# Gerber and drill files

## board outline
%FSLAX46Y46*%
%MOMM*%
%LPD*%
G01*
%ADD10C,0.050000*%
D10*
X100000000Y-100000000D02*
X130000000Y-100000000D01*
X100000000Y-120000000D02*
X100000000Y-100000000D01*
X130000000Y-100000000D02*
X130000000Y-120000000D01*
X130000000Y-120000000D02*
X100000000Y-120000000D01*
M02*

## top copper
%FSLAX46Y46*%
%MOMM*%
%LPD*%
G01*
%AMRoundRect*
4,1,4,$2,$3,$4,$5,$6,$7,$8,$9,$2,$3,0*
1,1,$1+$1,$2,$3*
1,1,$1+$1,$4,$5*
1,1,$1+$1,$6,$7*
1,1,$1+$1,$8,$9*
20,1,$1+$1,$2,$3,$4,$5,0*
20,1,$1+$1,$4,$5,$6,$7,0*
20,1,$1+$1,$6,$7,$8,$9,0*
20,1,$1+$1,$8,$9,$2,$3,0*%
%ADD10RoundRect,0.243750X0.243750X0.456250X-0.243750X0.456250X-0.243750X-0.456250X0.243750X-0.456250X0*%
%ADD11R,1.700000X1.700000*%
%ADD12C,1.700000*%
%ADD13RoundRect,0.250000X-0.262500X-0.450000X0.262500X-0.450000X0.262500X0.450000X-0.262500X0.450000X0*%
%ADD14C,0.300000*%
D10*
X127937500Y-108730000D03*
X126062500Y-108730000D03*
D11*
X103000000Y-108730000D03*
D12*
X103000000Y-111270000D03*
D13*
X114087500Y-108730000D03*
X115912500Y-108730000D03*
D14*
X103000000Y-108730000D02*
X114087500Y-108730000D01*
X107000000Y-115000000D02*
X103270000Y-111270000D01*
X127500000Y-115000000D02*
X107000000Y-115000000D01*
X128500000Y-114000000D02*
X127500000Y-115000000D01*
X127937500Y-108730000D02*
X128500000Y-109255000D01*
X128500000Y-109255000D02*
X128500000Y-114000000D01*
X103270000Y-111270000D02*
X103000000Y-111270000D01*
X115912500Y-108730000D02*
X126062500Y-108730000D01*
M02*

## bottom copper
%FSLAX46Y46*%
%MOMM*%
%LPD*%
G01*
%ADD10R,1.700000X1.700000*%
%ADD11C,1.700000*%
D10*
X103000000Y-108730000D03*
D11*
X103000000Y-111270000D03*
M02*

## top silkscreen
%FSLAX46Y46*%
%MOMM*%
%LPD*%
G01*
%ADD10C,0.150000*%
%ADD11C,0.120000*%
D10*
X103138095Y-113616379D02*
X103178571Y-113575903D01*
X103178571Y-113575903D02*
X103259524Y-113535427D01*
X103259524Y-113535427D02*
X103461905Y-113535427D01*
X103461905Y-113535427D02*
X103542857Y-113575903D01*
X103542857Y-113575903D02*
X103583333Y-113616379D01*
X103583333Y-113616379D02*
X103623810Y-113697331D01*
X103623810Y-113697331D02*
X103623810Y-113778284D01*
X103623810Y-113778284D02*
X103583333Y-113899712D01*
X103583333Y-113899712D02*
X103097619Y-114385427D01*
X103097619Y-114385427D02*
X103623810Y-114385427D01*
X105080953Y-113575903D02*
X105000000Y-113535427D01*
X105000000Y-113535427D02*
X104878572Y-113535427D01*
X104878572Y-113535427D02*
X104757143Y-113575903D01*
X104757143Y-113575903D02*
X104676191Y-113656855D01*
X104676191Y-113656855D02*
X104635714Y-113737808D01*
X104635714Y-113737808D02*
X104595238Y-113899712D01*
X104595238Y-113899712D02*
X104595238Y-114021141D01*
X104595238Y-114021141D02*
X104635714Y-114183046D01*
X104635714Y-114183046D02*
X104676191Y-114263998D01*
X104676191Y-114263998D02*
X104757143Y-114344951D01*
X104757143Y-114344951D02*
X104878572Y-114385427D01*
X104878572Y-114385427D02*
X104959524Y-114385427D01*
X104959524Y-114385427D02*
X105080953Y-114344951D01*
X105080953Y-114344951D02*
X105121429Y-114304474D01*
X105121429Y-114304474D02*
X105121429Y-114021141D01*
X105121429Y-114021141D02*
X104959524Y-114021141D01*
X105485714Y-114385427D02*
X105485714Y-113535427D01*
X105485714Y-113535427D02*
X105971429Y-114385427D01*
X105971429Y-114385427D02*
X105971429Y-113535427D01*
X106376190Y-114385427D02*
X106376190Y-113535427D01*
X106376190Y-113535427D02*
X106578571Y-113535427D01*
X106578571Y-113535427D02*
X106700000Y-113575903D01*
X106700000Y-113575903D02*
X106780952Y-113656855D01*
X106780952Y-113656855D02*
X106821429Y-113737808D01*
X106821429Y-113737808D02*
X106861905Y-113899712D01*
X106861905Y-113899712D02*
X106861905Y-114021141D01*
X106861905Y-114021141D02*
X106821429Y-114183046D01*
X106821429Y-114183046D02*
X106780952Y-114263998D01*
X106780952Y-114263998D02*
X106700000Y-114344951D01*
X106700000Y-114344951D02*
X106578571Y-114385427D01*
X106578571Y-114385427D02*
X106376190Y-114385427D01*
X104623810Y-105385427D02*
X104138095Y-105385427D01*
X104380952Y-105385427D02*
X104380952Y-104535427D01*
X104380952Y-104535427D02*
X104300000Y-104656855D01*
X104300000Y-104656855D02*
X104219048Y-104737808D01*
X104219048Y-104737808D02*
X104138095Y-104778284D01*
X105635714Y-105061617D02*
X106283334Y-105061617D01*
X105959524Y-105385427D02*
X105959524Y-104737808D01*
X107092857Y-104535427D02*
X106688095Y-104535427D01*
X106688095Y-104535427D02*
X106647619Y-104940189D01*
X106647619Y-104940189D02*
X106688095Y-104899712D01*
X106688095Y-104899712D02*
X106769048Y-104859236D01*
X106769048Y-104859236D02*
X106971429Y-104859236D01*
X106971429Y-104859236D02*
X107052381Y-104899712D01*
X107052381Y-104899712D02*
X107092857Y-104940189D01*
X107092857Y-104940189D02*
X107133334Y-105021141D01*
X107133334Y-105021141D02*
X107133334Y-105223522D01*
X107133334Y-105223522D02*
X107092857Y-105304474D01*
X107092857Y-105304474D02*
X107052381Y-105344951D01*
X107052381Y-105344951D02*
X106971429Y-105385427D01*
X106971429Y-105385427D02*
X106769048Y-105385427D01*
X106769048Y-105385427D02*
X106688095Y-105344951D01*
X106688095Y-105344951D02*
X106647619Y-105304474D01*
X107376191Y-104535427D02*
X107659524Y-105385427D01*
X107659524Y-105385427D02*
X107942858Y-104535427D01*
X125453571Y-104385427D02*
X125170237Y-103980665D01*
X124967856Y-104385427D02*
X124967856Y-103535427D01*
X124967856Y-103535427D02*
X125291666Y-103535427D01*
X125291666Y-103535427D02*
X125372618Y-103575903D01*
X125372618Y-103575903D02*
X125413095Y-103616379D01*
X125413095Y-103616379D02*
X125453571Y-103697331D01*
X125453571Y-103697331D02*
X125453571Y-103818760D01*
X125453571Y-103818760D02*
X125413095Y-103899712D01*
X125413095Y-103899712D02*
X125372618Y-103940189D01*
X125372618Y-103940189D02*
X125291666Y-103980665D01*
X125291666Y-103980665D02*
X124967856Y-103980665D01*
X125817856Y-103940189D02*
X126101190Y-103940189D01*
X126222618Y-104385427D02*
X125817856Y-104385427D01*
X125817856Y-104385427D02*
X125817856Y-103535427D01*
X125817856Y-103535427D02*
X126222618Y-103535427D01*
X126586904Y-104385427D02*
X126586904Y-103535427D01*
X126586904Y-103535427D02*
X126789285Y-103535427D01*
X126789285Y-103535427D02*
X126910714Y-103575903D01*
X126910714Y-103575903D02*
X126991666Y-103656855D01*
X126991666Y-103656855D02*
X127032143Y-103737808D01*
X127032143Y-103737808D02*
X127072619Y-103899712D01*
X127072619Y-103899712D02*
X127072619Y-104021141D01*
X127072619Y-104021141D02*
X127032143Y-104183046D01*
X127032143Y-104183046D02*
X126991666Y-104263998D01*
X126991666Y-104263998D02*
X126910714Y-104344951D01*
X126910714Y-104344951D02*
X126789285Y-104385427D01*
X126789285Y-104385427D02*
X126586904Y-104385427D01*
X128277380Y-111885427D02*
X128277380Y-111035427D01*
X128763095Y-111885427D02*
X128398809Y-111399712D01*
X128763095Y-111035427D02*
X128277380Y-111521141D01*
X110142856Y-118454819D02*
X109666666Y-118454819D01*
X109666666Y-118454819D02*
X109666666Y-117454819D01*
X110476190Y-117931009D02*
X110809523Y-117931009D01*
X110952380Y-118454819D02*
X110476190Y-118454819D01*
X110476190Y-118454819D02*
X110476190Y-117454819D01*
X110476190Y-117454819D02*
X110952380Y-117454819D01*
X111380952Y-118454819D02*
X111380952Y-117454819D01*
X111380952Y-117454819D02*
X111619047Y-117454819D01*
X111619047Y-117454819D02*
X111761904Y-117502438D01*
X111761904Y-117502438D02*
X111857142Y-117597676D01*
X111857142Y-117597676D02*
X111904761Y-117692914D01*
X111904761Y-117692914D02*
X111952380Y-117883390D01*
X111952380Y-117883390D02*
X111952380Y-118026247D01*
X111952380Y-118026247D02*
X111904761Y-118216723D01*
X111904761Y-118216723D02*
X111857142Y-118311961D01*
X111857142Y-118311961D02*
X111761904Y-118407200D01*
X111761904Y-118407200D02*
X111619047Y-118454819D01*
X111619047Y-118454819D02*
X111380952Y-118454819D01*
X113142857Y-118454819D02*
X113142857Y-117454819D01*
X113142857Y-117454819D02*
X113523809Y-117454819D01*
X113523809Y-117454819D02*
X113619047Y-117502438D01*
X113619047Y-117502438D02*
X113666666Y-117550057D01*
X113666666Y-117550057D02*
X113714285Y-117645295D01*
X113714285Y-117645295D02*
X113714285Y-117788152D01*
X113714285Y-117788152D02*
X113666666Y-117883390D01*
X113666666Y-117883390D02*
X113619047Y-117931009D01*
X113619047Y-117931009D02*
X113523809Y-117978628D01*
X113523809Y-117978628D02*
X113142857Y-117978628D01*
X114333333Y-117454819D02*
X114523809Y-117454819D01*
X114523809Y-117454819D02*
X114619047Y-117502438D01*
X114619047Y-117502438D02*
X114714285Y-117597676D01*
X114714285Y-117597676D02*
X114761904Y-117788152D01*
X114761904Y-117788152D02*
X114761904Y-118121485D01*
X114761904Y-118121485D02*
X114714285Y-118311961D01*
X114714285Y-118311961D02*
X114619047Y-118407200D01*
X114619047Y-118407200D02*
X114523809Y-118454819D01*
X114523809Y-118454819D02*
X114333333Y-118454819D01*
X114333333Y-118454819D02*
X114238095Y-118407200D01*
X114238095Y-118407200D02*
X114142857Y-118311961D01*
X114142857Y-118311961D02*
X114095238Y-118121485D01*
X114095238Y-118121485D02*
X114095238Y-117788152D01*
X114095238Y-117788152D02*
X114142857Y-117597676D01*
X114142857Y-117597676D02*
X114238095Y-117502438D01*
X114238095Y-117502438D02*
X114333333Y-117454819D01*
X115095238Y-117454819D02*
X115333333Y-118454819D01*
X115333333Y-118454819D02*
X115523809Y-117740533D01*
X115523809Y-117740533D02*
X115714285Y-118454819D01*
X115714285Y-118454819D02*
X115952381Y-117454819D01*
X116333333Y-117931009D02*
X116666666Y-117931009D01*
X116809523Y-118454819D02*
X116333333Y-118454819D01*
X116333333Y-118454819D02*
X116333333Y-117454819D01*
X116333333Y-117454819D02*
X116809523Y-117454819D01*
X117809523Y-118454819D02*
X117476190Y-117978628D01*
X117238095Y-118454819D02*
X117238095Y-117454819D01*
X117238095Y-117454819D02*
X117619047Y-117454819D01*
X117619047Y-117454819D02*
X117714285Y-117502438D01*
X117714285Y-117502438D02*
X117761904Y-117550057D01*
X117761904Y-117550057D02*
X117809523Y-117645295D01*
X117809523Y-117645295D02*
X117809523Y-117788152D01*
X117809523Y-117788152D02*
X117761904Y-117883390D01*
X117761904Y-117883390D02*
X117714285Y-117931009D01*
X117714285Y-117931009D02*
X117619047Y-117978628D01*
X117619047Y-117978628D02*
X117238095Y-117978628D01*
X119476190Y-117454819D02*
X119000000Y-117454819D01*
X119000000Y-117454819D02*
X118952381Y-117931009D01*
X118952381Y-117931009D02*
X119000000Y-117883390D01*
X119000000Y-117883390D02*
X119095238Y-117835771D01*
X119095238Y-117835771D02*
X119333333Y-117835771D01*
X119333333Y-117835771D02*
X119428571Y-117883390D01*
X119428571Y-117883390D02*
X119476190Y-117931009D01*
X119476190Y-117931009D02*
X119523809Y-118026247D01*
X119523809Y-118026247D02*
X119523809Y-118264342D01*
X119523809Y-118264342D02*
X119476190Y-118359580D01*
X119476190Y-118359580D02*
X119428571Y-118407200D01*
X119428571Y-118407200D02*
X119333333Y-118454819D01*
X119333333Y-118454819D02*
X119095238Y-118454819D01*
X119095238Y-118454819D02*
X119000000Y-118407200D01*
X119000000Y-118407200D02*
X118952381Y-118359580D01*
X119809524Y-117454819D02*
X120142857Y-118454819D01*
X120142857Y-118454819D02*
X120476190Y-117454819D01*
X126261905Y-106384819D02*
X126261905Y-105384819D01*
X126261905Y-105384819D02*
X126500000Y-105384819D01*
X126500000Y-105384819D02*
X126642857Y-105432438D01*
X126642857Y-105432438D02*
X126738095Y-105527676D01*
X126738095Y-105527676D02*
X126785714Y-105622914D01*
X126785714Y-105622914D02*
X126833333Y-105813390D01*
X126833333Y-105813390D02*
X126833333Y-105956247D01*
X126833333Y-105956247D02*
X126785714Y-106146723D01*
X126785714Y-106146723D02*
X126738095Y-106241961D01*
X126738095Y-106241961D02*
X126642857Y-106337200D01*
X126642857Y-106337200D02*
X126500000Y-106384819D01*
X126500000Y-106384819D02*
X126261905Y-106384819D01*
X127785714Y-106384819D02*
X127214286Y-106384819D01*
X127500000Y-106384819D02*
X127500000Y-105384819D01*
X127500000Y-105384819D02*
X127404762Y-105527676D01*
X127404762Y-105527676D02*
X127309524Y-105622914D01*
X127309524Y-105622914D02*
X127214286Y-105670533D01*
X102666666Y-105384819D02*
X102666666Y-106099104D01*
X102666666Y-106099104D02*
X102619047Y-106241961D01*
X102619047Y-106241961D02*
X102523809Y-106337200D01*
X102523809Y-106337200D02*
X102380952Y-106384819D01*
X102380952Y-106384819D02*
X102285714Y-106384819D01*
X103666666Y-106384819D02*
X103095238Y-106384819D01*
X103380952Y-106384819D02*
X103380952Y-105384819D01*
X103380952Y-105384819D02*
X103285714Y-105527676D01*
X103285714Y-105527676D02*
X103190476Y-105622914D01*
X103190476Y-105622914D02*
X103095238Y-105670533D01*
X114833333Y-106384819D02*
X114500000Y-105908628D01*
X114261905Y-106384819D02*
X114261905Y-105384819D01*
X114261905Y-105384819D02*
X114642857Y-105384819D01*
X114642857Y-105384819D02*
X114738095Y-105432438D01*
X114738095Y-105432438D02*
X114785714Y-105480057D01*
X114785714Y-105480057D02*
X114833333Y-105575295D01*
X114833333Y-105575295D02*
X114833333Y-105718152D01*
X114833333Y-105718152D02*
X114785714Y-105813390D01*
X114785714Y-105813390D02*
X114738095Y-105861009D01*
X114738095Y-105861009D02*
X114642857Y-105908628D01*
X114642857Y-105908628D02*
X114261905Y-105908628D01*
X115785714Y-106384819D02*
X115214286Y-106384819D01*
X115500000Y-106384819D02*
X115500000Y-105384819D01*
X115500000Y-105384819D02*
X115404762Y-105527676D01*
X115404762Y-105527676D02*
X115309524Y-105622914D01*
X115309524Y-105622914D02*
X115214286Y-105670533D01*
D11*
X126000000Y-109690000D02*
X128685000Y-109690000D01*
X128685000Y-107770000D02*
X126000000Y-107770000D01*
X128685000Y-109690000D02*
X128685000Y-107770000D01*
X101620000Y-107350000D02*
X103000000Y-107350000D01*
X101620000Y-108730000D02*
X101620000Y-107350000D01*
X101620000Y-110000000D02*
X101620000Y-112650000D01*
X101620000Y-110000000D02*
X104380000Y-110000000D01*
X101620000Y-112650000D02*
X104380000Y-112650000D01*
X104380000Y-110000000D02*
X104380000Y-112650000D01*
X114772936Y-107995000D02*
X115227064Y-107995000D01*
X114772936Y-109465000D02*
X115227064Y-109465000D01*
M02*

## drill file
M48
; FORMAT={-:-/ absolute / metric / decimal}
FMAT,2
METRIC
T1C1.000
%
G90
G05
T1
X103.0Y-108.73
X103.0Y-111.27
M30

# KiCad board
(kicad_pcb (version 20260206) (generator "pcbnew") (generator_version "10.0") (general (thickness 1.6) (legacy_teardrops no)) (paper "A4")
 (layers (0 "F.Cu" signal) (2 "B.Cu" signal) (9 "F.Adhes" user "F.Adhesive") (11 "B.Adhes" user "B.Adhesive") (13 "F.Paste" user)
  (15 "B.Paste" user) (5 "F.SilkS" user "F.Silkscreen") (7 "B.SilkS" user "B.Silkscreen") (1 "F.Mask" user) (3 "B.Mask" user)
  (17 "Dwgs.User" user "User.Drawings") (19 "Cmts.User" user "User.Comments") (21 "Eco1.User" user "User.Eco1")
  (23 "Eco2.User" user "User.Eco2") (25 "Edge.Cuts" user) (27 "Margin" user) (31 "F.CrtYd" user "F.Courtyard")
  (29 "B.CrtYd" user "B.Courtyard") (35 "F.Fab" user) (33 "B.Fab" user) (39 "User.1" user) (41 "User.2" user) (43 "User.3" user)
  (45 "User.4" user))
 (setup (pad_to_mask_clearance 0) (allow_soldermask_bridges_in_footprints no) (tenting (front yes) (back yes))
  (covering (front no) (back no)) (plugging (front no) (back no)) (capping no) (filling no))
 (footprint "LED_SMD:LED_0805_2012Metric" (layer "F.Cu") (at 127 108.73 180)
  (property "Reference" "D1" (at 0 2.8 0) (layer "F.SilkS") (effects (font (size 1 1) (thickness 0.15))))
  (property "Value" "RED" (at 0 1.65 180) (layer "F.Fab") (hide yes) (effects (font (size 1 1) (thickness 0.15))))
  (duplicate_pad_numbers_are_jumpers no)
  (fp_line (start 1 -0.96) (end -1.685 -0.96) (stroke (width 0.12) (type solid)) (layer "F.SilkS"))
  (fp_line (start -1.685 0.96) (end 1 0.96) (stroke (width 0.12) (type solid)) (layer "F.SilkS"))
  (fp_line (start -1.685 -0.96) (end -1.685 0.96) (stroke (width 0.12) (type solid)) (layer "F.SilkS"))
  (pad "1" smd roundrect (at -0.9375 0 180) (size 0.975 1.4) (layers "F.Cu" "F.Mask" "F.Paste") (roundrect_rratio 0.25) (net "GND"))
  (pad "2" smd roundrect (at 0.9375 0 180) (size 0.975 1.4) (layers "F.Cu" "F.Mask" "F.Paste") (roundrect_rratio 0.25) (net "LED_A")))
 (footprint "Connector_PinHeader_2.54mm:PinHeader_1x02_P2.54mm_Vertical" (layer "F.Cu") (at 103 108.73)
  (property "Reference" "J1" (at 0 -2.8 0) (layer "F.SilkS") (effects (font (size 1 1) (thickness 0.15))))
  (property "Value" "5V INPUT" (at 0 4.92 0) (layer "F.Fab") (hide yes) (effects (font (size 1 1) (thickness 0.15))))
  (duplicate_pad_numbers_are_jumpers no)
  (fp_line (start -1.38 -1.38) (end 0 -1.38) (stroke (width 0.12) (type solid)) (layer "F.SilkS"))
  (fp_line (start -1.38 0) (end -1.38 -1.38) (stroke (width 0.12) (type solid)) (layer "F.SilkS"))
  (fp_line (start -1.38 1.27) (end -1.38 3.92) (stroke (width 0.12) (type solid)) (layer "F.SilkS"))
  (fp_line (start -1.38 1.27) (end 1.38 1.27) (stroke (width 0.12) (type solid)) (layer "F.SilkS"))
  (fp_line (start -1.38 3.92) (end 1.38 3.92) (stroke (width 0.12) (type solid)) (layer "F.SilkS"))
  (fp_line (start 1.38 1.27) (end 1.38 3.92) (stroke (width 0.12) (type solid)) (layer "F.SilkS"))
  (pad "1" thru_hole rect (at 0 0) (size 1.7 1.7) (drill 1) (layers "*.Cu" "*.Mask") (remove_unused_layers no) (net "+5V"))
  (pad "2" thru_hole circle (at 0 2.54) (size 1.7 1.7) (drill 1) (layers "*.Cu" "*.Mask") (remove_unused_layers no) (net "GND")))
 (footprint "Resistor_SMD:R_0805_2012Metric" (layer "F.Cu") (at 115 108.73)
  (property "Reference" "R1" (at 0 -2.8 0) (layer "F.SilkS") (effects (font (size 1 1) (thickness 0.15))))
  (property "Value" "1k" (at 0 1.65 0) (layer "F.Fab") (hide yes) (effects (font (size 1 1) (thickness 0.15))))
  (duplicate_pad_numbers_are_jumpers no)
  (fp_line (start -0.227064 -0.735) (end 0.227064 -0.735) (stroke (width 0.12) (type solid)) (layer "F.SilkS"))
  (fp_line (start -0.227064 0.735) (end 0.227064 0.735) (stroke (width 0.12) (type solid)) (layer "F.SilkS"))
  (pad "1" smd roundrect (at -0.9125 0) (size 1.025 1.4) (layers "F.Cu" "F.Mask" "F.Paste") (roundrect_rratio 0.243902) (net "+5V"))
  (pad "2" smd roundrect (at 0.9125 0) (size 1.025 1.4) (layers "F.Cu" "F.Mask" "F.Paste") (roundrect_rratio 0.243902) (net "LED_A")))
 (gr_line (start 100 100) (end 130 100) (stroke (width 0.05) (type default)) (layer "Edge.Cuts"))
 (gr_line (start 100 120) (end 100 100) (stroke (width 0.05) (type default)) (layer "Edge.Cuts"))
 (gr_line (start 130 100) (end 130 120) (stroke (width 0.05) (type default)) (layer "Edge.Cuts"))
 (gr_line (start 130 120) (end 100 120) (stroke (width 0.05) (type default)) (layer "Edge.Cuts"))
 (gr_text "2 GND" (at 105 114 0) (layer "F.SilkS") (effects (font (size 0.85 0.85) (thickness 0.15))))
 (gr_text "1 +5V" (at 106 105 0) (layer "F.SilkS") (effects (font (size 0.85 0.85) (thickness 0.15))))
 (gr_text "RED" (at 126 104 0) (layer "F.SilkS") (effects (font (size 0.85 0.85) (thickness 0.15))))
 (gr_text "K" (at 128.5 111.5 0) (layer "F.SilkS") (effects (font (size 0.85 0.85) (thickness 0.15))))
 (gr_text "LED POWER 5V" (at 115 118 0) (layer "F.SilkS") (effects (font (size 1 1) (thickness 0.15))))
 (segment (start 103 108.73) (end 114.0875 108.73) (width 0.3) (layer "F.Cu") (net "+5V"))
 (segment (start 107 115) (end 103.27 111.27) (width 0.3) (layer "F.Cu") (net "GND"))
 (segment (start 127.5 115) (end 107 115) (width 0.3) (layer "F.Cu") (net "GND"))
 (segment (start 128.5 114) (end 127.5 115) (width 0.3) (layer "F.Cu") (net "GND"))
 (segment (start 127.9375 108.73) (end 128.5 109.255) (width 0.3) (layer "F.Cu") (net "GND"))
 (segment (start 128.5 109.255) (end 128.5 114) (width 0.3) (layer "F.Cu") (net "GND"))
 (segment (start 103.27 111.27) (end 103 111.27) (width 0.3) (layer "F.Cu") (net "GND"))
 (segment (start 115.9125 108.73) (end 126.0625 108.73) (width 0.3) (layer "F.Cu") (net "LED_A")))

